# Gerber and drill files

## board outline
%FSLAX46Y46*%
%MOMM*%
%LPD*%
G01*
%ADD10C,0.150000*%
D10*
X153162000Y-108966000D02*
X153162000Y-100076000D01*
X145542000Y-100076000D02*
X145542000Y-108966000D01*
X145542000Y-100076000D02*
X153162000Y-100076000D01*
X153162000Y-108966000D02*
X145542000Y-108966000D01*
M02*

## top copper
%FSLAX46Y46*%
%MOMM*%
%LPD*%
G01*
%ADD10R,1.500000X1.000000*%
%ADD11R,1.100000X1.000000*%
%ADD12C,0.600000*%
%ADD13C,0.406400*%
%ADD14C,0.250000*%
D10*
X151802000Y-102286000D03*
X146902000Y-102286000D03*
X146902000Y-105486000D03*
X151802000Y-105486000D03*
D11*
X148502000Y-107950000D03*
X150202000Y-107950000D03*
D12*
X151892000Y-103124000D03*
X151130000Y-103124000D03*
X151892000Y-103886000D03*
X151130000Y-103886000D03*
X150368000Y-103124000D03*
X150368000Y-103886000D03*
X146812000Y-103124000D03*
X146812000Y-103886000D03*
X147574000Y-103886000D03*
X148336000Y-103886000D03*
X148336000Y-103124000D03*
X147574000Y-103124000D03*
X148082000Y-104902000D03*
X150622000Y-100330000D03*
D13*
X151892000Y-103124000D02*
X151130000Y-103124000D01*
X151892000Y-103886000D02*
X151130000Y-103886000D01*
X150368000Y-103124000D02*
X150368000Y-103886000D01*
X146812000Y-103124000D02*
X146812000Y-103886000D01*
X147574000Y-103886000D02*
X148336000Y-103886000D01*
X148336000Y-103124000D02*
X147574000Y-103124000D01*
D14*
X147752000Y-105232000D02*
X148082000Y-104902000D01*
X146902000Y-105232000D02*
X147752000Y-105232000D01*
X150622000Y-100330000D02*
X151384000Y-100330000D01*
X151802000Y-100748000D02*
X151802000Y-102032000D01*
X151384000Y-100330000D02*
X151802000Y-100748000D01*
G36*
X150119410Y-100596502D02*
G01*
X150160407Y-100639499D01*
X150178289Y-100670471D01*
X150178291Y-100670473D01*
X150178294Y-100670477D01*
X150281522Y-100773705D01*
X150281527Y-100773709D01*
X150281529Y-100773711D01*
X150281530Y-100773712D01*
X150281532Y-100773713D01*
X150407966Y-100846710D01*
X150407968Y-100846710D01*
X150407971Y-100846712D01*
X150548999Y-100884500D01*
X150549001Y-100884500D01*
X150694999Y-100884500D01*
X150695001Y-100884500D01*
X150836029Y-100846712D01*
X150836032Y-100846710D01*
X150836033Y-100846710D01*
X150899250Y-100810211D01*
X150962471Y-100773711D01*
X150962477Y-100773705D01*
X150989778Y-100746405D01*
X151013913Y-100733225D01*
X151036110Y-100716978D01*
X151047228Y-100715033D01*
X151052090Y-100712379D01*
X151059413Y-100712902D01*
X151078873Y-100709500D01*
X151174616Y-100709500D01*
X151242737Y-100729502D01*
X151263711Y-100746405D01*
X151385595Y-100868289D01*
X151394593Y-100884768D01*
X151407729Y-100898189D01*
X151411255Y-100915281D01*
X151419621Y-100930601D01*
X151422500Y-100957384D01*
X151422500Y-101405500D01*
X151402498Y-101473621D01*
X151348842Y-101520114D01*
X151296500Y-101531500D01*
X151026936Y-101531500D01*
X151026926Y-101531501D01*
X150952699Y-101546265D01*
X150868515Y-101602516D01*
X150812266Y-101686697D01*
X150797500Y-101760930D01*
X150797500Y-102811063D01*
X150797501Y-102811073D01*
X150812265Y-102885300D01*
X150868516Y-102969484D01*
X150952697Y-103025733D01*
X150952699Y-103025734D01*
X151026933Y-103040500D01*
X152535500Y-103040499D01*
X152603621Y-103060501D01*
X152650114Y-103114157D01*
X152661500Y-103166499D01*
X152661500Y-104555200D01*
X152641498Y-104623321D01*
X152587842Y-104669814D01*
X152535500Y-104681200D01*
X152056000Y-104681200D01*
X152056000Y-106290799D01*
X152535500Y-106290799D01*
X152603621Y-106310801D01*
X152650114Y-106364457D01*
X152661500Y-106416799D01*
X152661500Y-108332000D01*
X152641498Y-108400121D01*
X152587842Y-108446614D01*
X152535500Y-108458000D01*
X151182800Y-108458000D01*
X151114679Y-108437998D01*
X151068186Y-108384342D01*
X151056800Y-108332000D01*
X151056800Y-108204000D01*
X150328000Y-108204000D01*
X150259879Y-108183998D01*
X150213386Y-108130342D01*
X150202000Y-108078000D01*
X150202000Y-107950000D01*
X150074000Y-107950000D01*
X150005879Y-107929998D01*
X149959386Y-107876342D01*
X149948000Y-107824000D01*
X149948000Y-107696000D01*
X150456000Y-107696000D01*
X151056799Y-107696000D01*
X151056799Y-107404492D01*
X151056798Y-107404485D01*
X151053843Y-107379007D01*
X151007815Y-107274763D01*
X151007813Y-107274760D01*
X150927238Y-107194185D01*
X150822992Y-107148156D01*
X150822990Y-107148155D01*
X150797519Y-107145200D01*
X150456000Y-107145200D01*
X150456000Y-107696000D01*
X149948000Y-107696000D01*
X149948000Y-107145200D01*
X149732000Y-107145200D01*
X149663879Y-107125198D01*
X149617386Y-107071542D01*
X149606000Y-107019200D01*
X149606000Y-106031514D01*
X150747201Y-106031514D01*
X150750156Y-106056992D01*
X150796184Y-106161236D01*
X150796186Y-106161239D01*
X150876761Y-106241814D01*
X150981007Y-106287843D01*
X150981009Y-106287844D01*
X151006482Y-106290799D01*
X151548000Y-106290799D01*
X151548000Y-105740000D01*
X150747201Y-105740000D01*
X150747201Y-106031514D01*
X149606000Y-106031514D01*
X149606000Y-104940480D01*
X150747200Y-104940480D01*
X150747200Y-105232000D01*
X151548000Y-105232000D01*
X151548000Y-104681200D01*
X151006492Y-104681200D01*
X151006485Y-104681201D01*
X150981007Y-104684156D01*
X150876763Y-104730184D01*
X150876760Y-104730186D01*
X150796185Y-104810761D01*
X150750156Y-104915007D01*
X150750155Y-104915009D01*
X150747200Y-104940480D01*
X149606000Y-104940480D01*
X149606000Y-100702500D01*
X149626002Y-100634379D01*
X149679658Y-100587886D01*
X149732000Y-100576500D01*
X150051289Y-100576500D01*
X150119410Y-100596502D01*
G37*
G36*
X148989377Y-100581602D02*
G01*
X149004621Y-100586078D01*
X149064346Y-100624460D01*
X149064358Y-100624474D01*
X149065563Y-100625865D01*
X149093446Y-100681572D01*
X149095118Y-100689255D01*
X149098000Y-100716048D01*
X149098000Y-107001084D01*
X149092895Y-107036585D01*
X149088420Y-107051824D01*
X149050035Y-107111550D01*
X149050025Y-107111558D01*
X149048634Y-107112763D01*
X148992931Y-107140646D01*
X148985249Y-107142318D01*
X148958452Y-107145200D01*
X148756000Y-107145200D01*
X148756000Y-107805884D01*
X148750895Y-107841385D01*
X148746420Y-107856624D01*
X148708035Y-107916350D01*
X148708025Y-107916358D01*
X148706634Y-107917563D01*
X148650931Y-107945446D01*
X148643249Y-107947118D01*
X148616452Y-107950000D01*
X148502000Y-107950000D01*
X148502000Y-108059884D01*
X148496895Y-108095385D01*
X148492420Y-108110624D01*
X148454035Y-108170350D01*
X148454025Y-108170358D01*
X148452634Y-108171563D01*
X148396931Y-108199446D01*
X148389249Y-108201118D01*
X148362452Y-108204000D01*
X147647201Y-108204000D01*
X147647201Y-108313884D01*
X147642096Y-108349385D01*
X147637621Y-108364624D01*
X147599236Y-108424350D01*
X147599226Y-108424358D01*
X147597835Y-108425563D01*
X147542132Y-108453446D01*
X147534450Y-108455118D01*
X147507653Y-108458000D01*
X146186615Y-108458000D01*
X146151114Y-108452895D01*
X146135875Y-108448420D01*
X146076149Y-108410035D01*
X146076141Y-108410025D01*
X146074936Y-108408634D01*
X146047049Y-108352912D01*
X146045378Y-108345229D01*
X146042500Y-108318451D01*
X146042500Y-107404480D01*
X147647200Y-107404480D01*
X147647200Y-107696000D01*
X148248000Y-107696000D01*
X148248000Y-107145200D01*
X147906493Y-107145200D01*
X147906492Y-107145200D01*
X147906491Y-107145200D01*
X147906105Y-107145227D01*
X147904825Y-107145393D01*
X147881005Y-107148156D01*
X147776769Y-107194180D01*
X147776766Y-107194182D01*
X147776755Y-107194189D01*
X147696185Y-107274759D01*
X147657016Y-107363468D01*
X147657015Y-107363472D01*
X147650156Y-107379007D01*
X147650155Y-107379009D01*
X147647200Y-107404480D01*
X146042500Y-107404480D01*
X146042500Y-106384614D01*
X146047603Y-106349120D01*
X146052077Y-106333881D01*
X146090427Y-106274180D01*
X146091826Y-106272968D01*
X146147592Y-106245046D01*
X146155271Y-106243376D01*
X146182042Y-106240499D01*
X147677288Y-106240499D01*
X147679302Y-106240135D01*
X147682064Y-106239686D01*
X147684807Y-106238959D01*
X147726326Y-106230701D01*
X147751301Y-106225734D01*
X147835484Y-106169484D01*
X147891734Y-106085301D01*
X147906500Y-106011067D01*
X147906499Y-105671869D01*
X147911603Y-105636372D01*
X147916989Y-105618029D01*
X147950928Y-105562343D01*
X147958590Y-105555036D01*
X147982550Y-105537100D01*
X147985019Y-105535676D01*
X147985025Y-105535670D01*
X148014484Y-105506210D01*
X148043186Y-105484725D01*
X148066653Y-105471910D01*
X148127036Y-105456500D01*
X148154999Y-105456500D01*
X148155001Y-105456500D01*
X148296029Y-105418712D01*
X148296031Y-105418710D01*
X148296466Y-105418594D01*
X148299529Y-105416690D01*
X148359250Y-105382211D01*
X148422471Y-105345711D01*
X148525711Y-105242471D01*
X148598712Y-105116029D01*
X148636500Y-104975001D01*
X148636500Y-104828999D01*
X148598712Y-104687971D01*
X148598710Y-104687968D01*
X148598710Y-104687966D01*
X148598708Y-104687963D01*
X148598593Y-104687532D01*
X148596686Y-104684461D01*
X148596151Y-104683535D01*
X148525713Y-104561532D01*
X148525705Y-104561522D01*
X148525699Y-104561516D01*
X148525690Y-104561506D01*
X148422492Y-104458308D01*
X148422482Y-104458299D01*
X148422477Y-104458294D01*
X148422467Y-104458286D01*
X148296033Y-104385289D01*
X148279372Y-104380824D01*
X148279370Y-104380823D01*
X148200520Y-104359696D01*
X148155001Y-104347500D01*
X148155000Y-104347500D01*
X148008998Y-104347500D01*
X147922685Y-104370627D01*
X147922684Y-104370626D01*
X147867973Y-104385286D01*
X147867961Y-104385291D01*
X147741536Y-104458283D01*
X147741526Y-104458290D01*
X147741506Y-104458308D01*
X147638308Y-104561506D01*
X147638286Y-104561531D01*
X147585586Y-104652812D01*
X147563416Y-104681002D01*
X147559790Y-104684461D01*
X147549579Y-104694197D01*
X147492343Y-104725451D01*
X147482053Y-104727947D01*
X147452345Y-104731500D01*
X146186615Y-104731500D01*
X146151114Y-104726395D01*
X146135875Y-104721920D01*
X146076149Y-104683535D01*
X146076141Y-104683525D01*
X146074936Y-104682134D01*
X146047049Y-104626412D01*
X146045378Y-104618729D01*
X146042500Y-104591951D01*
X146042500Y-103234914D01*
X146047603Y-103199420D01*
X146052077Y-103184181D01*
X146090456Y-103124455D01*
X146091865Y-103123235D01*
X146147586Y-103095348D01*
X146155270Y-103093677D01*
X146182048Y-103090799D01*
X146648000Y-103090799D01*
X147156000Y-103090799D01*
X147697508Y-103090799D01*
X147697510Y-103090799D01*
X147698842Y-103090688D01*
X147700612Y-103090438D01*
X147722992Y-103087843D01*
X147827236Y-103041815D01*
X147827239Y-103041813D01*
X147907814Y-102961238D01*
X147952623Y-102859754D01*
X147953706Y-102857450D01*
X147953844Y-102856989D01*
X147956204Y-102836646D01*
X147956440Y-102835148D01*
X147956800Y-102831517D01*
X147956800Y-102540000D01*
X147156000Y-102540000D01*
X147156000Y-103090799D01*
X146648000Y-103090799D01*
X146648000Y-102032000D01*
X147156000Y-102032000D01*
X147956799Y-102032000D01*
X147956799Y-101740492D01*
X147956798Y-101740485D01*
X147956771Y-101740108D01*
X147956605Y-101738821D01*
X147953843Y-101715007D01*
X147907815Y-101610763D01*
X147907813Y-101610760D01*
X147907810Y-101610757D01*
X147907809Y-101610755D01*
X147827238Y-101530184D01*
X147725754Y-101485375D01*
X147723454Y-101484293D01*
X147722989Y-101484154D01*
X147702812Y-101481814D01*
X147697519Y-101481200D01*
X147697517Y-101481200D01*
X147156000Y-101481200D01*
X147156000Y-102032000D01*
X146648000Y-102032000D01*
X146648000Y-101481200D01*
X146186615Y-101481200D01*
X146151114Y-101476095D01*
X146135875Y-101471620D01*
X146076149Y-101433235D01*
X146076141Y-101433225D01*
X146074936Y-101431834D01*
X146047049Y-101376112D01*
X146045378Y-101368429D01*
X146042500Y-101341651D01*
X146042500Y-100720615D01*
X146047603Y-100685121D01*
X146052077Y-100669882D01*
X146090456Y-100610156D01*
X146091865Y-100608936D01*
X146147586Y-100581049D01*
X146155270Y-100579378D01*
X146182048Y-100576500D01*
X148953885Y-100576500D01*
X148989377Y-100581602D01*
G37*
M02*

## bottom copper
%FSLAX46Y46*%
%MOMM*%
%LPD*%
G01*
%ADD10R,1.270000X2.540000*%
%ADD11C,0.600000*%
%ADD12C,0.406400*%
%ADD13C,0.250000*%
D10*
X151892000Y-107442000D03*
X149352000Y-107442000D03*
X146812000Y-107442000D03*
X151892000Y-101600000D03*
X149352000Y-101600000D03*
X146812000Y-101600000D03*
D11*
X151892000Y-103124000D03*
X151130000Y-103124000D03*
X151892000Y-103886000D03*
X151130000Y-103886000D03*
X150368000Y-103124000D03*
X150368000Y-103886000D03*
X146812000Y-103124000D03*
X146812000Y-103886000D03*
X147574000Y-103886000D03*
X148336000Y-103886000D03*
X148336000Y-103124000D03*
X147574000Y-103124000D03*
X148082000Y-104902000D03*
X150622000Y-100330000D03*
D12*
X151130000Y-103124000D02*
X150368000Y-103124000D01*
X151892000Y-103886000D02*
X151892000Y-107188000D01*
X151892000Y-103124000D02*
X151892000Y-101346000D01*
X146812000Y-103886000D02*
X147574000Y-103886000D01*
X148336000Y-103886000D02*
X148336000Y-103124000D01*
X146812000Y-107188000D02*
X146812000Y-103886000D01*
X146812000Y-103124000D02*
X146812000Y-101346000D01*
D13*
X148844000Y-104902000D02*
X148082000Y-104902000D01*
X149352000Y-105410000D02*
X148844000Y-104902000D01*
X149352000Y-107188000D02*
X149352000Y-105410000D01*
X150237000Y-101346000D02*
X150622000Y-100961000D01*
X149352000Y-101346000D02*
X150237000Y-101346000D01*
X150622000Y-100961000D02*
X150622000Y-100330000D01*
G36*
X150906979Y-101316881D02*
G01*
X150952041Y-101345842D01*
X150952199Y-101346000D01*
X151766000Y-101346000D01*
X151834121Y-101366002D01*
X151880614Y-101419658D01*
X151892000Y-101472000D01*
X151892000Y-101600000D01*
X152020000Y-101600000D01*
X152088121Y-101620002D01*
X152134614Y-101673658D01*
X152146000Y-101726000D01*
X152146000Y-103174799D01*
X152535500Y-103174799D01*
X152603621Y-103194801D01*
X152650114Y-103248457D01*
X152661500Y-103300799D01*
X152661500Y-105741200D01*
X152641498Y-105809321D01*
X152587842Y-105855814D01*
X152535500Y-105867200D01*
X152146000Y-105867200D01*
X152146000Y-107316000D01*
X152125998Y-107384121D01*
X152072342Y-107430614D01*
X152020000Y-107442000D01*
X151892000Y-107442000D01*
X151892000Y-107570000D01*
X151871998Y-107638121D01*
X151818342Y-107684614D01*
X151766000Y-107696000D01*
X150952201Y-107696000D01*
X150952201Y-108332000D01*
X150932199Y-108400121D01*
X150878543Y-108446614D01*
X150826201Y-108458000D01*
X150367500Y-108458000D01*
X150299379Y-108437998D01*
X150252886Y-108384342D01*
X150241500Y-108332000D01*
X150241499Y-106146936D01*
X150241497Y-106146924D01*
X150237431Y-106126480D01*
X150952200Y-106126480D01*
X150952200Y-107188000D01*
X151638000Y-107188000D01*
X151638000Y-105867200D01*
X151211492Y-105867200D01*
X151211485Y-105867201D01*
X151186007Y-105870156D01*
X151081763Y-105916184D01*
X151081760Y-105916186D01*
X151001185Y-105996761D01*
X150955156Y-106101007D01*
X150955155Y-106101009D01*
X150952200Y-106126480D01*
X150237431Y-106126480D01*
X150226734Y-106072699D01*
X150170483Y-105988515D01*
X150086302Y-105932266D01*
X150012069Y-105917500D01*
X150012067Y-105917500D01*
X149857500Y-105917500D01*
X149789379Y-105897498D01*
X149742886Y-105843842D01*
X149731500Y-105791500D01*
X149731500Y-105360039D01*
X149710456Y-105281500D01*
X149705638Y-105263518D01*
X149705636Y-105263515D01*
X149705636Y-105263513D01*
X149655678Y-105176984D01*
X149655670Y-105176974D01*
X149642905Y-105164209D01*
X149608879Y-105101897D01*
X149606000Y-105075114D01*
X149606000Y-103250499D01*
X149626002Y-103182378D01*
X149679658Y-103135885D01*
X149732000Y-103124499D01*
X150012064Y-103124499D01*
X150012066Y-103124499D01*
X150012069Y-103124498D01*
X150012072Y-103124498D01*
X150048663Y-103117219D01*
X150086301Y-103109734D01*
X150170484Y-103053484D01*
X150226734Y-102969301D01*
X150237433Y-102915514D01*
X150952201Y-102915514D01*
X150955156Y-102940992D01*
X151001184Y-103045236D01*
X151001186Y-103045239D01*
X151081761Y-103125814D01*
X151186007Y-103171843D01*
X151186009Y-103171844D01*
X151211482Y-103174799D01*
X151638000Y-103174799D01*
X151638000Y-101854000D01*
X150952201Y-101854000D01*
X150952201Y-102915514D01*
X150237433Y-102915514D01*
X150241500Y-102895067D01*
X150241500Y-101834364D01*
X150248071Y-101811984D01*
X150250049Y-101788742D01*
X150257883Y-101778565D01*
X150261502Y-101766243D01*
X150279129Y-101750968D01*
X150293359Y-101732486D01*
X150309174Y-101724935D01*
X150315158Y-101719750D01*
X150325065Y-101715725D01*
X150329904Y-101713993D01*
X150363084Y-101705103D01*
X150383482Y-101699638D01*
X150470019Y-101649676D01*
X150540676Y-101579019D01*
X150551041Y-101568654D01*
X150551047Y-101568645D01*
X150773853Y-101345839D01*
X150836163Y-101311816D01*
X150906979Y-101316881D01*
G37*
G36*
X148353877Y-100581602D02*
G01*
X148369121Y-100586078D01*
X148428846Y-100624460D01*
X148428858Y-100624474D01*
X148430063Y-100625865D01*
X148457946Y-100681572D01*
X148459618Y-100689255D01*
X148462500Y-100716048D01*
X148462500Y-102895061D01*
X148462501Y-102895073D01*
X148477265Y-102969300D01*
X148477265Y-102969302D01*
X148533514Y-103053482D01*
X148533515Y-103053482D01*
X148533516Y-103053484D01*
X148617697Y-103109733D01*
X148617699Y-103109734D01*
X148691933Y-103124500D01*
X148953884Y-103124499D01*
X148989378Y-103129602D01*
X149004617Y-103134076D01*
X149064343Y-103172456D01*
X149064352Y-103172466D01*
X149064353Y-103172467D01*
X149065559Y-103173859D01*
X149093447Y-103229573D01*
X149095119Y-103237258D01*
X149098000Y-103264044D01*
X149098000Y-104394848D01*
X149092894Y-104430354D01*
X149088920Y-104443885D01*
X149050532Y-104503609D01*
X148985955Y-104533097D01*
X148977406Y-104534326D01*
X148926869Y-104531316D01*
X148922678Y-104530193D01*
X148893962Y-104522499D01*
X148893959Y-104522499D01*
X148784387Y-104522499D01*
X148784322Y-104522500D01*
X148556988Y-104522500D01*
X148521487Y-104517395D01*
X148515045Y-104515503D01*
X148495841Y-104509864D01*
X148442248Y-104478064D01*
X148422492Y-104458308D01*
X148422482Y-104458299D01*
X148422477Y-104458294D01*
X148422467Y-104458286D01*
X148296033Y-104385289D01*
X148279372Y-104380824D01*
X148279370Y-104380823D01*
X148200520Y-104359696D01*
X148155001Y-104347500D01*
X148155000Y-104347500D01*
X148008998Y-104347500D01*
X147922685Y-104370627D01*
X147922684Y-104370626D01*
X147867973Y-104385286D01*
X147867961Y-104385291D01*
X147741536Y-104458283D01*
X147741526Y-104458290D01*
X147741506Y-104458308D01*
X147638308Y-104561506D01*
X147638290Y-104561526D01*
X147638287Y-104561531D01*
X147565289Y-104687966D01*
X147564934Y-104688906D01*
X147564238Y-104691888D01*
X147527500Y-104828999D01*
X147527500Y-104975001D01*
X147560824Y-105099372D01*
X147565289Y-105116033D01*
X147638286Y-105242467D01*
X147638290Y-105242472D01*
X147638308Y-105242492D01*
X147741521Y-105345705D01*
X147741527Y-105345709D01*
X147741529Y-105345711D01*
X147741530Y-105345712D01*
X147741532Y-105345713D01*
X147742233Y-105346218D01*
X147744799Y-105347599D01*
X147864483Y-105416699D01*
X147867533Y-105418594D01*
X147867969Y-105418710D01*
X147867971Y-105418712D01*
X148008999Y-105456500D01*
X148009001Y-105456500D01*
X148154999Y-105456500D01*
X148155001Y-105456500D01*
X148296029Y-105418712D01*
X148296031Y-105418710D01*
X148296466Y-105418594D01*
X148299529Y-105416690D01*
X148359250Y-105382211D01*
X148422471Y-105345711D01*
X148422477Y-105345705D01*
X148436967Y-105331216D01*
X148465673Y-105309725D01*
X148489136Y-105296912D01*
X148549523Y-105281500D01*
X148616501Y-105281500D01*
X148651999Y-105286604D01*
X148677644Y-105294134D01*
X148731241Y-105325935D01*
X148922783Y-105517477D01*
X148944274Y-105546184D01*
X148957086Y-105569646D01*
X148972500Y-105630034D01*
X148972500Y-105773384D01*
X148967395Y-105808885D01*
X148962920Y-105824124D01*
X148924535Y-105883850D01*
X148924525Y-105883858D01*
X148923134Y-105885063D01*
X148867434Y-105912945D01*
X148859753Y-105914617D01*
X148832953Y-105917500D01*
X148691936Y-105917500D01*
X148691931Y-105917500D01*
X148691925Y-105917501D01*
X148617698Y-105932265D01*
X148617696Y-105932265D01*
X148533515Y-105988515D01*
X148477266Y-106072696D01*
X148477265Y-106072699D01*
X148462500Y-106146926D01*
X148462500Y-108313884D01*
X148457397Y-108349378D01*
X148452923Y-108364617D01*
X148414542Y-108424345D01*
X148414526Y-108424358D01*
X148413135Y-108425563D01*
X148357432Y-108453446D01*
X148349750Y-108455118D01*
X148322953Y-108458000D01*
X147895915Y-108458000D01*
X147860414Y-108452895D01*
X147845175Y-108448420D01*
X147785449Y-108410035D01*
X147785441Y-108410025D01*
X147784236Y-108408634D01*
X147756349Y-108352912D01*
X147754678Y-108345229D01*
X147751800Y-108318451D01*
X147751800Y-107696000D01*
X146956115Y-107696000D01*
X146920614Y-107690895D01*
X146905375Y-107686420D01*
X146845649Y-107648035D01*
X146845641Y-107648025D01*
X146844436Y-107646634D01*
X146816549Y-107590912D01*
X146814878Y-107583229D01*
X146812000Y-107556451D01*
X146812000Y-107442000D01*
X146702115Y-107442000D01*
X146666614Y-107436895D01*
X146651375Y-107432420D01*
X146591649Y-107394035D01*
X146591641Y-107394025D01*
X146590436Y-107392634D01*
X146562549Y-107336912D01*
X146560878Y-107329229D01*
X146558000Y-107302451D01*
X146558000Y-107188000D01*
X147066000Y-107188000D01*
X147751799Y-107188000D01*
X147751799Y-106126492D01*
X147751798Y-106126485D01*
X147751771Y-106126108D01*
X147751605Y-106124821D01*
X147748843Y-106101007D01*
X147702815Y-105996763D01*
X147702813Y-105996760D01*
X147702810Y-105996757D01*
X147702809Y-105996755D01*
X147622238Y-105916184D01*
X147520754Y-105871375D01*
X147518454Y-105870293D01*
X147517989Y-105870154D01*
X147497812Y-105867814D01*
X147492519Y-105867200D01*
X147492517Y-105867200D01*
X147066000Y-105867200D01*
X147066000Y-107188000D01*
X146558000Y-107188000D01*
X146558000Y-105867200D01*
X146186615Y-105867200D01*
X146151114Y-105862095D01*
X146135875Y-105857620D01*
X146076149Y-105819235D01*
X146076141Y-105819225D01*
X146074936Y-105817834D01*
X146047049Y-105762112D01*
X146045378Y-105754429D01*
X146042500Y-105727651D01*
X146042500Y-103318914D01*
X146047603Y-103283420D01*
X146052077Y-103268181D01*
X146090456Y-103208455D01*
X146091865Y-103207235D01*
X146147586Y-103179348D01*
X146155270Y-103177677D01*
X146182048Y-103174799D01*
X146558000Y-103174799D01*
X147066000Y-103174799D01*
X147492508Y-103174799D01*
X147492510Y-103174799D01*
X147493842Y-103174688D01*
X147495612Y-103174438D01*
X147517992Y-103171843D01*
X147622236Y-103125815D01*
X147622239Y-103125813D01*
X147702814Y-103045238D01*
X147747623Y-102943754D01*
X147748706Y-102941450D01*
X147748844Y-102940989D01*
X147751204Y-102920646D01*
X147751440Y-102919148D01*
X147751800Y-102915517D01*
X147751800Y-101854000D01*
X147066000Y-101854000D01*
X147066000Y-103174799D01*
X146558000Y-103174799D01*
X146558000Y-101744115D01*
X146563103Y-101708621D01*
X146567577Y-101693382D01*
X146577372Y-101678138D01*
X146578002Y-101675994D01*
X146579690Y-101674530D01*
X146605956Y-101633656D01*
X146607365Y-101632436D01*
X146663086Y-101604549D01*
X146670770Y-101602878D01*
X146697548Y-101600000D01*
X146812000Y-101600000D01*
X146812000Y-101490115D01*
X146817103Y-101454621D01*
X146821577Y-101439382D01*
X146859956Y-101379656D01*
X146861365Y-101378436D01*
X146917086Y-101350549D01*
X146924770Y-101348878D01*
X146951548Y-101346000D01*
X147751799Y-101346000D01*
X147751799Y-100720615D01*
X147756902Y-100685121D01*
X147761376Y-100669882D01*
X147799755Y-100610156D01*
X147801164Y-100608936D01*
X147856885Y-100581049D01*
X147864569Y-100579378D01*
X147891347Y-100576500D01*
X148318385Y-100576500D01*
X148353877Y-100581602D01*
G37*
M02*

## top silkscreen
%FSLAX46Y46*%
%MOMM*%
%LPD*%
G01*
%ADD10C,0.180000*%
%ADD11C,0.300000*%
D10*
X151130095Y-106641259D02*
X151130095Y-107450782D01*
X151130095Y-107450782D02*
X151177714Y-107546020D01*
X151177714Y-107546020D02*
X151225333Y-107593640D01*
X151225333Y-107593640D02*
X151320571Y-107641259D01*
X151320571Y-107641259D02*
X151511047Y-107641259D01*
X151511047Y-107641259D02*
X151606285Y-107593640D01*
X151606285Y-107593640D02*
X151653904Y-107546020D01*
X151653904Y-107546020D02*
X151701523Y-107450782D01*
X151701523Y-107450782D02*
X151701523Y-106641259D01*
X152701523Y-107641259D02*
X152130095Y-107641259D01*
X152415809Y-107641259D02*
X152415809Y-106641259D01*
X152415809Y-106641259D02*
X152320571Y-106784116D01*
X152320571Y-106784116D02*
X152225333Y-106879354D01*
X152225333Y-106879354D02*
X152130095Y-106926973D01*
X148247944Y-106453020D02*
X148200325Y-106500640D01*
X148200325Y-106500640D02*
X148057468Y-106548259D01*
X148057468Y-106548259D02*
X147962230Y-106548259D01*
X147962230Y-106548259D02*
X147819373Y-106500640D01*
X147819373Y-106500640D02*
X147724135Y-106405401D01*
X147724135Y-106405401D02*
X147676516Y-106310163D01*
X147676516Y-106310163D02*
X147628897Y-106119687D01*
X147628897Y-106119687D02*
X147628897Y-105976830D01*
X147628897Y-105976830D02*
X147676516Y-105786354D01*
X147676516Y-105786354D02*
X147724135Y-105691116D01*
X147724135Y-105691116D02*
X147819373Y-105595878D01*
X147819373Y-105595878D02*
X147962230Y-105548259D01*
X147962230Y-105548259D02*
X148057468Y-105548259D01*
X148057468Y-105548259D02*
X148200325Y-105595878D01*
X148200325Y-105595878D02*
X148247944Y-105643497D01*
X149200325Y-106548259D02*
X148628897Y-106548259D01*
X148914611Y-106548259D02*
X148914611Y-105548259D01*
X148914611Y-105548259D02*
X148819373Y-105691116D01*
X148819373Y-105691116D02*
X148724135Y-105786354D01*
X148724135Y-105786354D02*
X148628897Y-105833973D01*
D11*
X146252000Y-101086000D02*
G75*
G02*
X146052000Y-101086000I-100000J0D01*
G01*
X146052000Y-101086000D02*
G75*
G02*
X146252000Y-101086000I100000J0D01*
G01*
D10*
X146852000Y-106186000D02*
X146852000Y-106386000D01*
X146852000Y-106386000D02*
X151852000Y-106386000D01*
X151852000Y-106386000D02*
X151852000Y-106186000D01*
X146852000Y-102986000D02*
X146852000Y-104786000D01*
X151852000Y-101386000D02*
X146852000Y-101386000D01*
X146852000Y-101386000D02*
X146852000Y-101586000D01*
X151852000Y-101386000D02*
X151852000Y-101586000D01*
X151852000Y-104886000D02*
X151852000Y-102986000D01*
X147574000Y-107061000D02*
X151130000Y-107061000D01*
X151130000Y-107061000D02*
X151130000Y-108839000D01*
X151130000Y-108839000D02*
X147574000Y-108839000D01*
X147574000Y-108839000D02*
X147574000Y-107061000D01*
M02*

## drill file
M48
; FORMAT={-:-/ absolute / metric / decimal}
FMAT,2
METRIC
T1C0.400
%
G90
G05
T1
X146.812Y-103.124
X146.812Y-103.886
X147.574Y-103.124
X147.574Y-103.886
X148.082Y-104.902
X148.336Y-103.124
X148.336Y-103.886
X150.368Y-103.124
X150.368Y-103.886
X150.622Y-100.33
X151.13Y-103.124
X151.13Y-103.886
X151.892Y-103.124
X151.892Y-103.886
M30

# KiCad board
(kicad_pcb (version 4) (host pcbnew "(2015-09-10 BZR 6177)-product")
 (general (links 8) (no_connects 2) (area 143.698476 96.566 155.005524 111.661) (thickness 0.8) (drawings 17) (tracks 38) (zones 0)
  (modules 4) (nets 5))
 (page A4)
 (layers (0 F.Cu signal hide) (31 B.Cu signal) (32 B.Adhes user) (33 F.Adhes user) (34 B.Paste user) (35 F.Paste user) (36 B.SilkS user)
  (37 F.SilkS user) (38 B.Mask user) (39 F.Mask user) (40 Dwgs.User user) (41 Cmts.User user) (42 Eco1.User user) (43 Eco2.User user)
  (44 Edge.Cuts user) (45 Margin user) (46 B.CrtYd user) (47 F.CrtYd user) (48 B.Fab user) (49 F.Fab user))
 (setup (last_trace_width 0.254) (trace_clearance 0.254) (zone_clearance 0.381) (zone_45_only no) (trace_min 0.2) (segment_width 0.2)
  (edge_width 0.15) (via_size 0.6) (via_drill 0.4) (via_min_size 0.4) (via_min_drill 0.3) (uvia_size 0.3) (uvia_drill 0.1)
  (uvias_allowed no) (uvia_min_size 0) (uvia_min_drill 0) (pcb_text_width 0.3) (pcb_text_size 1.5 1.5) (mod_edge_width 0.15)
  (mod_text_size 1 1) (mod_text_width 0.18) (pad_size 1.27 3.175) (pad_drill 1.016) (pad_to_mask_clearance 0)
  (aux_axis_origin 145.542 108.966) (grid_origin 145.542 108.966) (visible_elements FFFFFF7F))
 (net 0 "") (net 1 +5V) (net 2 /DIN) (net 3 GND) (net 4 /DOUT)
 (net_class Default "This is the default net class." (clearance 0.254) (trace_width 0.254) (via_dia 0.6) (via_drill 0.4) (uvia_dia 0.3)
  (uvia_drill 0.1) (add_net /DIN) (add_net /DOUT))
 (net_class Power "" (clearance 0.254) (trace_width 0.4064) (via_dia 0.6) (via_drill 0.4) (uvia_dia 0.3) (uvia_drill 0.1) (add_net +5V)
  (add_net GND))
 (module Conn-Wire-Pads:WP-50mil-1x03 (layer B.Cu) (at 149.352 107.442 180)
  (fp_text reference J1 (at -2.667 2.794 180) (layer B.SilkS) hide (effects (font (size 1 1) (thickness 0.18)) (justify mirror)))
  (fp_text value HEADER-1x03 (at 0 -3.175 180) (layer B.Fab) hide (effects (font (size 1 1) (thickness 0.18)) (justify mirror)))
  (pad 1 smd rect (at -2.54 0 180) (size 1.27 2.54) (layers B.Cu B.Paste B.Mask) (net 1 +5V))
  (pad 2 smd rect (at 0 0 180) (size 1.27 2.54) (layers B.Cu B.Paste B.Mask) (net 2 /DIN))
  (pad 3 smd rect (at 2.54 0 180) (size 1.27 2.54) (layers B.Cu B.Paste B.Mask) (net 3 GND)))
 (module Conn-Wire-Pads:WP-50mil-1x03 (layer B.Cu) (at 149.352 101.6 180)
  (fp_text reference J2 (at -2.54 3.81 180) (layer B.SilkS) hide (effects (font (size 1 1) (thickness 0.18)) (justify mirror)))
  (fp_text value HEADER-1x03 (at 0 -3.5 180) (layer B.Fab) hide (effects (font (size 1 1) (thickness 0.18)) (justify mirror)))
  (pad 1 smd rect (at -2.54 0 180) (size 1.27 2.54) (layers B.Cu B.Paste B.Mask) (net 1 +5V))
  (pad 2 smd rect (at 0 0 180) (size 1.27 2.54) (layers B.Cu B.Paste B.Mask) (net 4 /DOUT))
  (pad 3 smd rect (at 2.54 0 180) (size 1.27 2.54) (layers B.Cu B.Paste B.Mask) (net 3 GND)))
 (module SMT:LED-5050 (layer F.Cu) (at 149.352 103.886 180)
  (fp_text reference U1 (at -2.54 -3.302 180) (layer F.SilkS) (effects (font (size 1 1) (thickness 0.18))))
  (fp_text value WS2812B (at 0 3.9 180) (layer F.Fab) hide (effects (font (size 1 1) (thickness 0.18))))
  (fp_circle (center 3.2 2.8) (end 3.3 2.8) (layer F.SilkS) (width 0.3))
  (fp_line (start 2.5 -2.3) (end 2.5 -2.5) (layer F.SilkS) (width 0.18))
  (fp_line (start 2.5 -2.5) (end -2.5 -2.5) (layer F.SilkS) (width 0.18))
  (fp_line (start -2.5 -2.5) (end -2.5 -2.3) (layer F.SilkS) (width 0.18))
  (fp_line (start 2.5 0.9) (end 2.5 -0.9) (layer F.SilkS) (width 0.18))
  (fp_line (start -2.5 2.5) (end 2.5 2.5) (layer F.SilkS) (width 0.18))
  (fp_line (start 2.5 2.5) (end 2.5 2.3) (layer F.SilkS) (width 0.18))
  (fp_line (start -2.5 2.5) (end -2.5 2.3) (layer F.SilkS) (width 0.18))
  (fp_line (start -2.5 -1) (end -2.5 0.9) (layer F.SilkS) (width 0.18))
  (pad 2 smd rect (at -2.45 1.6 180) (size 1.5 1) (layers F.Cu F.Paste F.Mask) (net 4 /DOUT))
  (pad 3 smd rect (at 2.45 1.6 180) (size 1.5 1) (layers F.Cu F.Paste F.Mask) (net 3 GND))
  (pad 4 smd rect (at 2.45 -1.6 180) (size 1.5 1) (layers F.Cu F.Paste F.Mask) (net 2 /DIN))
  (pad 1 smd rect (at -2.45 -1.6 180) (size 1.5 1) (layers F.Cu F.Paste F.Mask) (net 1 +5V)))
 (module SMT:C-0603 (layer F.Cu) (at 149.352 107.95)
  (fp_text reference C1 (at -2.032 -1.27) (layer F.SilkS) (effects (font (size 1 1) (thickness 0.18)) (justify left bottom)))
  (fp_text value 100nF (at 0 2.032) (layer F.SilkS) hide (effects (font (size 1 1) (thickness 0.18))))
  (fp_line (start -1.778 -0.889) (end 1.778 -0.889) (layer F.SilkS) (width 0.18))
  (fp_line (start 1.778 -0.889) (end 1.778 0.889) (layer F.SilkS) (width 0.18))
  (fp_line (start 1.778 0.889) (end -1.778 0.889) (layer F.SilkS) (width 0.18))
  (fp_line (start -1.778 0.889) (end -1.778 -0.889) (layer F.SilkS) (width 0.18))
  (pad 1 smd rect (at -0.85 0) (size 1.1 1) (layers F.Cu F.Paste F.Mask) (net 3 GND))
  (pad 2 smd rect (at 0.85 0) (size 1.1 1) (layers F.Cu F.Paste F.Mask) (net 1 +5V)))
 (gr_line (start 153.162 108.966) (end 153.162 100.076) (angle 90) (layer Edge.Cuts) (width 0.15))
 (gr_line (start 145.542 100.076) (end 145.542 108.966) (angle 90) (layer Edge.Cuts) (width 0.15))
 (gr_line (start 145.542 100.076) (end 153.162 100.076) (angle 90) (layer Edge.Cuts) (width 0.15))
 (gr_line (start 153.162 108.966) (end 145.542 108.966) (angle 90) (layer Edge.Cuts) (width 0.15))
 (via (at 151.892 103.124) (size 0.6) (drill 0.4) (layers F.Cu B.Cu) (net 1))
 (via (at 151.13 103.124) (size 0.6) (drill 0.4) (layers F.Cu B.Cu) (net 1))
 (segment (start 151.892 103.124) (end 151.13 103.124) (width 0.4064) (layer F.Cu) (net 1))
 (via (at 151.892 103.886) (size 0.6) (drill 0.4) (layers F.Cu B.Cu) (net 1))
 (via (at 151.13 103.886) (size 0.6) (drill 0.4) (layers F.Cu B.Cu) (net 1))
 (segment (start 151.892 103.886) (end 151.13 103.886) (width 0.4064) (layer F.Cu) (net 1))
 (via (at 150.368 103.124) (size 0.6) (drill 0.4) (layers F.Cu B.Cu) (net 1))
 (segment (start 151.13 103.124) (end 150.368 103.124) (width 0.4064) (layer B.Cu) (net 1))
 (via (at 150.368 103.886) (size 0.6) (drill 0.4) (layers F.Cu B.Cu) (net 1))
 (segment (start 150.368 103.124) (end 150.368 103.886) (width 0.4064) (layer F.Cu) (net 1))
 (segment (start 151.892 103.886) (end 151.892 107.188) (width 0.4064) (layer B.Cu) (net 1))
 (segment (start 151.892 103.124) (end 151.892 101.346) (width 0.4064) (layer B.Cu) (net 1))
 (via (at 146.812 103.124) (size 0.6) (drill 0.4) (layers F.Cu B.Cu) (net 3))
 (via (at 146.812 103.886) (size 0.6) (drill 0.4) (layers F.Cu B.Cu) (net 3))
 (segment (start 146.812 103.124) (end 146.812 103.886) (width 0.4064) (layer F.Cu) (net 3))
 (via (at 147.574 103.886) (size 0.6) (drill 0.4) (layers F.Cu B.Cu) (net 3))
 (segment (start 146.812 103.886) (end 147.574 103.886) (width 0.4064) (layer B.Cu) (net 3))
 (via (at 148.336 103.886) (size 0.6) (drill 0.4) (layers F.Cu B.Cu) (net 3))
 (segment (start 147.574 103.886) (end 148.336 103.886) (width 0.4064) (layer F.Cu) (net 3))
 (via (at 148.336 103.124) (size 0.6) (drill 0.4) (layers F.Cu B.Cu) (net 3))
 (segment (start 148.336 103.886) (end 148.336 103.124) (width 0.4064) (layer B.Cu) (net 3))
 (via (at 147.574 103.124) (size 0.6) (drill 0.4) (layers F.Cu B.Cu) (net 3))
 (segment (start 148.336 103.124) (end 147.574 103.124) (width 0.4064) (layer F.Cu) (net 3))
 (segment (start 146.812 107.188) (end 146.812 103.886) (width 0.4064) (layer B.Cu) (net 3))
 (segment (start 146.812 103.124) (end 146.812 101.346) (width 0.4064) (layer B.Cu) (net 3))
 (via (at 148.082 104.902) (size 0.6) (drill 0.4) (layers F.Cu B.Cu) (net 2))
 (segment (start 147.752 105.232) (end 148.082 104.902) (width 0.25) (layer F.Cu) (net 2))
 (segment (start 146.902 105.232) (end 147.752 105.232) (width 0.25) (layer F.Cu) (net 2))
 (segment (start 148.844 104.902) (end 148.082 104.902) (width 0.25) (layer B.Cu) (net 2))
 (segment (start 149.352 105.41) (end 148.844 104.902) (width 0.25) (layer B.Cu) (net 2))
 (segment (start 149.352 107.188) (end 149.352 105.41) (width 0.25) (layer B.Cu) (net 2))
 (via (at 150.622 100.33) (size 0.6) (drill 0.4) (layers F.Cu B.Cu) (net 4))
 (segment (start 150.622 100.33) (end 151.384 100.33) (width 0.25) (layer F.Cu) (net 4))
 (segment (start 151.802 100.748) (end 151.802 102.032) (width 0.25) (layer F.Cu) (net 4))
 (segment (start 151.384 100.33) (end 151.802 100.748) (width 0.25) (layer F.Cu) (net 4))
 (segment (start 150.237 101.346) (end 150.622 100.961) (width 0.25) (layer B.Cu) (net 4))
 (segment (start 149.352 101.346) (end 150.237 101.346) (width 0.25) (layer B.Cu) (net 4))
 (segment (start 150.622 100.961) (end 150.622 100.33) (width 0.25) (layer B.Cu) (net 4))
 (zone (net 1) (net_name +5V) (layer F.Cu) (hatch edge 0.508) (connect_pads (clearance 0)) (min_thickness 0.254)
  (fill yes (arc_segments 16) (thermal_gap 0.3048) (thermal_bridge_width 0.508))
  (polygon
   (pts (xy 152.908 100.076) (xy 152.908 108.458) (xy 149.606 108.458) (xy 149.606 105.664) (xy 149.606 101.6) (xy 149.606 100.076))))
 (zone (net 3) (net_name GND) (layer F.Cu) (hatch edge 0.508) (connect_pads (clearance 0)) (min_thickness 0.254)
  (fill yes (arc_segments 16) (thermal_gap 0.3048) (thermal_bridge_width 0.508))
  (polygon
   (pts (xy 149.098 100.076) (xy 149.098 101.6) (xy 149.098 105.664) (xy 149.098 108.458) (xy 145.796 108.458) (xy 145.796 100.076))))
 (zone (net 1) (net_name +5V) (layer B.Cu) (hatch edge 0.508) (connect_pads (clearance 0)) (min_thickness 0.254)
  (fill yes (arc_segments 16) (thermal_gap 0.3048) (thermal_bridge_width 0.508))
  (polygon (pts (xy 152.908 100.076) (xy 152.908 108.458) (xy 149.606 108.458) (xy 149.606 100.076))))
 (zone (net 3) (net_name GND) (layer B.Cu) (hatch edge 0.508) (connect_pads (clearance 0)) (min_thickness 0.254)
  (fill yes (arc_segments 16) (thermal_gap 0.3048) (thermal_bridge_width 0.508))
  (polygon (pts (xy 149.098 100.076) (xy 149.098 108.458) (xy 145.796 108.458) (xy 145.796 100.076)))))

